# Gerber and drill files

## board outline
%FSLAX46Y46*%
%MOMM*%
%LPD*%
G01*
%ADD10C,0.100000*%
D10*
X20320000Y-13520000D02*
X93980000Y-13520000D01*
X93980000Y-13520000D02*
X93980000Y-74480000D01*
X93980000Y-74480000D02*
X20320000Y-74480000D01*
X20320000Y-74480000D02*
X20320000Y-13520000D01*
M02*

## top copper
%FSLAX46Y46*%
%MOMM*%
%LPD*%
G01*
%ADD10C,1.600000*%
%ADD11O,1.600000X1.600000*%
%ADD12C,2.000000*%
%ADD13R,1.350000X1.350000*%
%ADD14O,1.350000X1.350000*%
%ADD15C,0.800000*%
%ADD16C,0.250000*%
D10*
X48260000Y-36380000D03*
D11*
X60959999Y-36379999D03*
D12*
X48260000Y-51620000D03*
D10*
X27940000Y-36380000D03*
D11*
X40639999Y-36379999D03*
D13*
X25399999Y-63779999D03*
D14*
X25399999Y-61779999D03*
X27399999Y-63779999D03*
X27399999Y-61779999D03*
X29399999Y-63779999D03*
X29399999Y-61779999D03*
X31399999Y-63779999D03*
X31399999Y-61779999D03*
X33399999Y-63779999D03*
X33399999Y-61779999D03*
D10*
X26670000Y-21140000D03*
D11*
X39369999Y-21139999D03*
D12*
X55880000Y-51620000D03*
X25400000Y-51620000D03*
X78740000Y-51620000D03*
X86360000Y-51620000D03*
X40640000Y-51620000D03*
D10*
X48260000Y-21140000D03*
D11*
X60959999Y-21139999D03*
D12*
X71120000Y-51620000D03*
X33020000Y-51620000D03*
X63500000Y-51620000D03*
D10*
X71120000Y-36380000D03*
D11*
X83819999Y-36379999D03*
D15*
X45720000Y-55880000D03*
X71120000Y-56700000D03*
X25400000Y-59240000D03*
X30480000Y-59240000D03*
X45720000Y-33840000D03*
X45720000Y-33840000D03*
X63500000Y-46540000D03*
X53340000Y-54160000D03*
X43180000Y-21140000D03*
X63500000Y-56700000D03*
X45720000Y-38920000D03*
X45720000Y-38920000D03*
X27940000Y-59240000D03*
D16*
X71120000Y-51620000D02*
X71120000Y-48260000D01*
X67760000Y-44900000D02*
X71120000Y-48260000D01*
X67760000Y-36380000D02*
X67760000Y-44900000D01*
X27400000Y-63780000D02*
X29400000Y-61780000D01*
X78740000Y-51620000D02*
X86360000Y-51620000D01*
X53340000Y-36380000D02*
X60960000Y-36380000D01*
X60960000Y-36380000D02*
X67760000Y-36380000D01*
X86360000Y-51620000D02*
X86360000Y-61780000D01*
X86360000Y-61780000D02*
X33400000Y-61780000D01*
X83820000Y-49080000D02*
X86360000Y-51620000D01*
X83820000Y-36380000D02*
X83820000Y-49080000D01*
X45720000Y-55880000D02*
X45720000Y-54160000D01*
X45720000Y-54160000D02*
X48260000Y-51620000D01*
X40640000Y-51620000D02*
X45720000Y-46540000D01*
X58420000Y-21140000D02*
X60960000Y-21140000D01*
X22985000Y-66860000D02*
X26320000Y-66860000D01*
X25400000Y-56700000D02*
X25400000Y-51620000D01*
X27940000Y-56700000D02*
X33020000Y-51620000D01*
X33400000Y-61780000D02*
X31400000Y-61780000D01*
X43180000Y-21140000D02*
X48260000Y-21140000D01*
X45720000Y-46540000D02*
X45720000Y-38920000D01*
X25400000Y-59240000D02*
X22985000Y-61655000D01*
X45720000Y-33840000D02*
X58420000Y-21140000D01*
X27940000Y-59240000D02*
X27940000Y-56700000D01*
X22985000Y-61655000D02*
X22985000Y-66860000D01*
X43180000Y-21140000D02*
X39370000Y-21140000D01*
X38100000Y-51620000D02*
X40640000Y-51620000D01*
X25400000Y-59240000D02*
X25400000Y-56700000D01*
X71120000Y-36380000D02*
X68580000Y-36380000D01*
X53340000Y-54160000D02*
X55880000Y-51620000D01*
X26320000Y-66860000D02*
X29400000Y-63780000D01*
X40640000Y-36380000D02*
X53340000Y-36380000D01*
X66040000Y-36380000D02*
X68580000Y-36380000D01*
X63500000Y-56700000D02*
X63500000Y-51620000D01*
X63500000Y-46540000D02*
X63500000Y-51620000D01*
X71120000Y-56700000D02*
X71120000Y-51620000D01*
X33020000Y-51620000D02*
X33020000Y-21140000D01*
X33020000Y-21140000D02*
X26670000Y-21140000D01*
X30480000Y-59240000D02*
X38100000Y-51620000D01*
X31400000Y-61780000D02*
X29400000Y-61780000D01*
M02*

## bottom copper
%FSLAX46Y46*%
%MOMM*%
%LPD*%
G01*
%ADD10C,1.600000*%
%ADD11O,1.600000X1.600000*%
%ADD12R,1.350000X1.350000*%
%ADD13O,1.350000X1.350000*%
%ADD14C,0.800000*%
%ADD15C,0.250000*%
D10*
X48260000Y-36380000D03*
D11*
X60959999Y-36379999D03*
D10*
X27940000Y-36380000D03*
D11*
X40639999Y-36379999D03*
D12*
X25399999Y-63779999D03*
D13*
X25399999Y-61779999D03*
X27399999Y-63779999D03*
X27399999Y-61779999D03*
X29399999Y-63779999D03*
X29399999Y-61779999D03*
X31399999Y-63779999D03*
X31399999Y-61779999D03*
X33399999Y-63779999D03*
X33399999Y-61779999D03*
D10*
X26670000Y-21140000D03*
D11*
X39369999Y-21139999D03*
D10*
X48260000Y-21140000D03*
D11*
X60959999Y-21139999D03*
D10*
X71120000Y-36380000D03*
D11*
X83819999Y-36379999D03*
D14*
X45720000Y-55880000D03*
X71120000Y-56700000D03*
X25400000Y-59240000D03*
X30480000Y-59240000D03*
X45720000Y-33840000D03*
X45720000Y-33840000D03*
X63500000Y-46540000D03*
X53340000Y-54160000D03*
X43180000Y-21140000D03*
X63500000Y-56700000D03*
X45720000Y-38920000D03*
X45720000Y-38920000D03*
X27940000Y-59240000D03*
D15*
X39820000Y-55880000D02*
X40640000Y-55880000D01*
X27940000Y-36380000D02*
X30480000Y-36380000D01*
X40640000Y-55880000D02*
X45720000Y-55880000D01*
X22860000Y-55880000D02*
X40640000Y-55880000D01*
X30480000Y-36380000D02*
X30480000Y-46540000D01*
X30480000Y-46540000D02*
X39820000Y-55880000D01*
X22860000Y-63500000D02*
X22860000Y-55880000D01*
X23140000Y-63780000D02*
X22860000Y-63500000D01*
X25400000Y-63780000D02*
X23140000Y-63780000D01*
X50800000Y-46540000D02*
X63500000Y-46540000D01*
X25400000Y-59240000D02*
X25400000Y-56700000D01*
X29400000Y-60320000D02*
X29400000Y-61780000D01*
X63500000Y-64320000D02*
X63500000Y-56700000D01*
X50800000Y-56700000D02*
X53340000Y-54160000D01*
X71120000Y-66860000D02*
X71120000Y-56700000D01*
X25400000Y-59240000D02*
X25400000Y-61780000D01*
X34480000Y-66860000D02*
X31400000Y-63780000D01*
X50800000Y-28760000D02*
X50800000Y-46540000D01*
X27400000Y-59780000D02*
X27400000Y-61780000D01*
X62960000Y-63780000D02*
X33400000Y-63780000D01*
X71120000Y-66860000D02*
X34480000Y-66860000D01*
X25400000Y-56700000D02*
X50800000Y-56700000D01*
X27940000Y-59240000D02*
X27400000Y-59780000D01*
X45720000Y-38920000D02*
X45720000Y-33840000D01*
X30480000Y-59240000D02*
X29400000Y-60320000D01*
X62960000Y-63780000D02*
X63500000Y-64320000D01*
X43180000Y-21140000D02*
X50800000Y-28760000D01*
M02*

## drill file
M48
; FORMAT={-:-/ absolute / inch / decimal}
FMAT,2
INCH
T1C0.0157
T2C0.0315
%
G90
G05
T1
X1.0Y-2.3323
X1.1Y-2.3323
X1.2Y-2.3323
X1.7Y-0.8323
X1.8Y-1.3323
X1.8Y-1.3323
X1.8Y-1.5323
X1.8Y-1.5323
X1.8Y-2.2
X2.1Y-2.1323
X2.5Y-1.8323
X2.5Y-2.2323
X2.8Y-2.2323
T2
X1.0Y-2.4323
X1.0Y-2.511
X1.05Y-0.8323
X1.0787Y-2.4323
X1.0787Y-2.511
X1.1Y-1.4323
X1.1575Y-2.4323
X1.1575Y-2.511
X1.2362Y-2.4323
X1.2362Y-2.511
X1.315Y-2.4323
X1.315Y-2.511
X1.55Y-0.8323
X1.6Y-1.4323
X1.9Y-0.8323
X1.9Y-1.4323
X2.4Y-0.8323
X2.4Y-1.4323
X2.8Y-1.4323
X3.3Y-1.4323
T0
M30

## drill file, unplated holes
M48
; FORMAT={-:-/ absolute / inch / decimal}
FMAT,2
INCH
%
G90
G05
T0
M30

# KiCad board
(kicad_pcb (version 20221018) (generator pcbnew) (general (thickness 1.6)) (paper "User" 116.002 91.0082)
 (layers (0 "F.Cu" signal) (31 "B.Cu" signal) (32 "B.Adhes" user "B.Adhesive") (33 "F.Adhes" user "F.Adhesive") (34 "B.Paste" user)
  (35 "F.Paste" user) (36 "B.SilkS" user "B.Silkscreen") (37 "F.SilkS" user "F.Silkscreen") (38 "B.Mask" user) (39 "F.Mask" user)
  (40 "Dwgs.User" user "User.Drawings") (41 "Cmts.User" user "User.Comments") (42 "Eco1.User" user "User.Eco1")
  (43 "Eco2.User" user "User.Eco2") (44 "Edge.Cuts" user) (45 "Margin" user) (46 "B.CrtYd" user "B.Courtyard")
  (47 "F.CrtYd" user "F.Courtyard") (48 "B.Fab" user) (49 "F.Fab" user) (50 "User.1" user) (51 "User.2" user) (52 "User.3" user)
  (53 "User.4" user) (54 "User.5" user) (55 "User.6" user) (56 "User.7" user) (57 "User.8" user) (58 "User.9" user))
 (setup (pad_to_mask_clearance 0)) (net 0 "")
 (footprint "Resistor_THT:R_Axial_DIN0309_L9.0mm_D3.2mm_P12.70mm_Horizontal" (layer "F.Cu") (at 27.94 36.38)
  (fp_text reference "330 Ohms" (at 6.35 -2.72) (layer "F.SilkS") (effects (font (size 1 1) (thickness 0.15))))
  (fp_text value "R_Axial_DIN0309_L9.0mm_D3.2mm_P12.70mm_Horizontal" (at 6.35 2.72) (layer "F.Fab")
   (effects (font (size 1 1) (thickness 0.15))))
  (pad "1" thru_hole circle (at 0 0) (size 1.6 1.6) (drill 0.8) (layers "*.Cu" "*.Mask"))
  (pad "2" thru_hole oval (at 12.7 0) (size 1.6 1.6) (drill 0.8) (layers "*.Cu" "*.Mask")))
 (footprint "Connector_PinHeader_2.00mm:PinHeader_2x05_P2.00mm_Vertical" (layer "F.Cu") (at 25.4 63.78 90)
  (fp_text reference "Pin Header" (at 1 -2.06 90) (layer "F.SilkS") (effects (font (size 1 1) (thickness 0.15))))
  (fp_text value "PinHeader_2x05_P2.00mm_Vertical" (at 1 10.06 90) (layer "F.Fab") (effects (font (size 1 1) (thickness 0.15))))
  (pad "1" thru_hole rect (at 0 0 90) (size 1.35 1.35) (drill 0.8) (layers "*.Cu" "*.Mask"))
  (pad "2" thru_hole oval (at 2 0 90) (size 1.35 1.35) (drill 0.8) (layers "*.Cu" "*.Mask"))
  (pad "3" thru_hole oval (at 0 2 90) (size 1.35 1.35) (drill 0.8) (layers "*.Cu" "*.Mask"))
  (pad "4" thru_hole oval (at 2 2 90) (size 1.35 1.35) (drill 0.8) (layers "*.Cu" "*.Mask"))
  (pad "5" thru_hole oval (at 0 4 90) (size 1.35 1.35) (drill 0.8) (layers "*.Cu" "*.Mask"))
  (pad "6" thru_hole oval (at 2 4 90) (size 1.35 1.35) (drill 0.8) (layers "*.Cu" "*.Mask"))
  (pad "7" thru_hole oval (at 0 6 90) (size 1.35 1.35) (drill 0.8) (layers "*.Cu" "*.Mask"))
  (pad "8" thru_hole oval (at 2 6 90) (size 1.35 1.35) (drill 0.8) (layers "*.Cu" "*.Mask"))
  (pad "9" thru_hole oval (at 0 8 90) (size 1.35 1.35) (drill 0.8) (layers "*.Cu" "*.Mask"))
  (pad "10" thru_hole oval (at 2 8 90) (size 1.35 1.35) (drill 0.8) (layers "*.Cu" "*.Mask")))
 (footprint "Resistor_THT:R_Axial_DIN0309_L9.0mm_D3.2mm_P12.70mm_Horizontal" (layer "F.Cu") (at 26.67 21.14)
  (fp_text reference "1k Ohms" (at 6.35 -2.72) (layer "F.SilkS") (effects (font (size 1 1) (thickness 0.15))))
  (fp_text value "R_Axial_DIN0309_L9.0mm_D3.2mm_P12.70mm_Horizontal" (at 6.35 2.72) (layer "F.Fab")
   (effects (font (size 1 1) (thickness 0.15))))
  (pad "1" thru_hole circle (at 0 0) (size 1.6 1.6) (drill 0.8) (layers "*.Cu" "*.Mask"))
  (pad "2" thru_hole oval (at 12.7 0) (size 1.6 1.6) (drill 0.8) (layers "*.Cu" "*.Mask")))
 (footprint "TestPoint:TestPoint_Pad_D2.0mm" (layer "F.Cu") (at 55.88 51.62)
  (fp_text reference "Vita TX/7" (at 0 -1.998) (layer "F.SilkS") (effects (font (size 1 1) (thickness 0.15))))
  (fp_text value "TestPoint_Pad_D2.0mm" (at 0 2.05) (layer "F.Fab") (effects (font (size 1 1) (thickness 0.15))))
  (pad "1" smd circle (at 0 0) (size 2 2) (layers "F.Cu" "F.Mask")))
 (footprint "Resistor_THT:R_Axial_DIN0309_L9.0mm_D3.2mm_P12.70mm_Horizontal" (layer "F.Cu") (at 48.26 36.38)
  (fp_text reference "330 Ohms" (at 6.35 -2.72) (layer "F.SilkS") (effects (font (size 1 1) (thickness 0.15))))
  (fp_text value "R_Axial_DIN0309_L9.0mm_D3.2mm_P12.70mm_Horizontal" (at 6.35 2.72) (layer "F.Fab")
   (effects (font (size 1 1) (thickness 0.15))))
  (pad "1" thru_hole circle (at 0 0) (size 1.6 1.6) (drill 0.8) (layers "*.Cu" "*.Mask"))
  (pad "2" thru_hole oval (at 12.7 0) (size 1.6 1.6) (drill 0.8) (layers "*.Cu" "*.Mask")))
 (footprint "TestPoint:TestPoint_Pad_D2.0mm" (layer "F.Cu") (at 48.26 51.62)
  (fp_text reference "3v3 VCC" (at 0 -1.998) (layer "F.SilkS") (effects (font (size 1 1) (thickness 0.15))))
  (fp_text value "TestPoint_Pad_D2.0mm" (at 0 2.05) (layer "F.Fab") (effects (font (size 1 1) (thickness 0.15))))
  (pad "1" smd circle (at 0 0) (size 2 2) (layers "F.Cu" "F.Mask")))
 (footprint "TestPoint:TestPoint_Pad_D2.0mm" (layer "F.Cu") (at 25.4 51.62)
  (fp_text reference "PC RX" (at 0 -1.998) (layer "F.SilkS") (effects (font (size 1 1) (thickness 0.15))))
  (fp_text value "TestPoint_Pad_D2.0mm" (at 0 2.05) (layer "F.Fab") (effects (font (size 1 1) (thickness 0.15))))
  (pad "1" smd circle (at 0 0) (size 2 2) (layers "F.Cu" "F.Mask")))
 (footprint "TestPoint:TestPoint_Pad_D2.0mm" (layer "F.Cu") (at 78.74 51.62)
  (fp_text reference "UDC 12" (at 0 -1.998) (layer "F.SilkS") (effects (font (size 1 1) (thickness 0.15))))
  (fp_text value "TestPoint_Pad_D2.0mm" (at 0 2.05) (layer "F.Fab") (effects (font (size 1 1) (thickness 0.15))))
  (pad "1" smd circle (at 0 0) (size 2 2) (layers "F.Cu" "F.Mask")))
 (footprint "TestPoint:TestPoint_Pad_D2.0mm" (layer "F.Cu") (at 86.36 51.62)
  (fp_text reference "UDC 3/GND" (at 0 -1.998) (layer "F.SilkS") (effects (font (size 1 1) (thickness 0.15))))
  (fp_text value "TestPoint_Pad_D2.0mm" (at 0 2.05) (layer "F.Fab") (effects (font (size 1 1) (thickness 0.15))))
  (pad "1" smd circle (at 0 0) (size 2 2) (layers "F.Cu" "F.Mask")))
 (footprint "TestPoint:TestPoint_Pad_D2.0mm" (layer "F.Cu") (at 40.64 51.62)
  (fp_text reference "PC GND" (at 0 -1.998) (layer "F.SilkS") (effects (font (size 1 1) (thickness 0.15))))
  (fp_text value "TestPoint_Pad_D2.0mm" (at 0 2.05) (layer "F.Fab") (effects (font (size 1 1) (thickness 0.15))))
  (pad "1" smd circle (at 0 0) (size 2 2) (layers "F.Cu" "F.Mask")))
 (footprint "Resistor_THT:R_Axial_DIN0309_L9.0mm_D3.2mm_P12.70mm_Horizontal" (layer "F.Cu") (at 48.26 21.14)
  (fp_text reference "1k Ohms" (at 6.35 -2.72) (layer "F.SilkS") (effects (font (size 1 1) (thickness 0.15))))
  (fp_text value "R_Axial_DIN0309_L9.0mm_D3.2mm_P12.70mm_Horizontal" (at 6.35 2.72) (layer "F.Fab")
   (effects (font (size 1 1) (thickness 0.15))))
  (pad "1" thru_hole circle (at 0 0) (size 1.6 1.6) (drill 0.8) (layers "*.Cu" "*.Mask"))
  (pad "2" thru_hole oval (at 12.7 0) (size 1.6 1.6) (drill 0.8) (layers "*.Cu" "*.Mask")))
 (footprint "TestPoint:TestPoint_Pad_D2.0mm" (layer "F.Cu") (at 71.12 51.62)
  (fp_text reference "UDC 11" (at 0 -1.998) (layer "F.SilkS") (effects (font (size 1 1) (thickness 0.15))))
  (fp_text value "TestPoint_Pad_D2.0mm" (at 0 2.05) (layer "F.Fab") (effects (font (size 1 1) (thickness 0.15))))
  (pad "1" smd circle (at 0 0) (size 2 2) (layers "F.Cu" "F.Mask")))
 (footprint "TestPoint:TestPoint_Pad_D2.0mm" (layer "F.Cu") (at 33.02 51.62)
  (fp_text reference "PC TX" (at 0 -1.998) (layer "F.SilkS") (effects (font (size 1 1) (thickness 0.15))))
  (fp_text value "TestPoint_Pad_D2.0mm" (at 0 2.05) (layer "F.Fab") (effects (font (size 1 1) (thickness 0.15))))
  (pad "1" smd circle (at 0 0) (size 2 2) (layers "F.Cu" "F.Mask")))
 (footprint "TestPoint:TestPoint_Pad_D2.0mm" (layer "F.Cu") (at 63.5 51.62)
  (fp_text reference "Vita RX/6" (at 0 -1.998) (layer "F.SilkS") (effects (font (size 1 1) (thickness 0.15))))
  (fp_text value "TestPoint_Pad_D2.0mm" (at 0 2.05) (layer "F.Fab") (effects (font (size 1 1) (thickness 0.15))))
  (pad "1" smd circle (at 0 0) (size 2 2) (layers "F.Cu" "F.Mask")))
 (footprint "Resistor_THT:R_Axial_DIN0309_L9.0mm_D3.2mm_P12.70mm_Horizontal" (layer "F.Cu") (at 71.12 36.38)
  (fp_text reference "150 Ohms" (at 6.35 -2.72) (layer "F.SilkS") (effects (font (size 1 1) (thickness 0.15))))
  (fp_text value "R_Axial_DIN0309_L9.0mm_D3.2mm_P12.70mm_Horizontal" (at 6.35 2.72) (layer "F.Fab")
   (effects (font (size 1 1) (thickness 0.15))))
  (pad "1" thru_hole circle (at 0 0) (size 1.6 1.6) (drill 0.8) (layers "*.Cu" "*.Mask"))
  (pad "2" thru_hole oval (at 12.7 0) (size 1.6 1.6) (drill 0.8) (layers "*.Cu" "*.Mask")))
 (gr_rect (start 20.32 13.52) (end 93.98 74.48) (stroke (width 0.1) (type default)) (fill none) (layer "Edge.Cuts"))
 (segment (start 67.76 36.38) (end 67.76 44.9) (width 0.25) (layer "F.Cu") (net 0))
 (segment (start 40.64 51.62) (end 45.72 46.54) (width 0.25) (layer "F.Cu") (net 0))
 (segment (start 58.42 21.14) (end 60.96 21.14) (width 0.25) (layer "F.Cu") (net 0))
 (segment (start 22.985 66.86) (end 26.32 66.86) (width 0.25) (layer "F.Cu") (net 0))
 (segment (start 25.4 56.7) (end 25.4 51.62) (width 0.25) (layer "F.Cu") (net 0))
 (segment (start 83.82 49.08) (end 86.36 51.62) (width 0.25) (layer "F.Cu") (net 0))
 (segment (start 27.94 56.7) (end 33.02 51.62) (width 0.25) (layer "F.Cu") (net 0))
 (segment (start 33.4 61.78) (end 31.4 61.78) (width 0.25) (layer "F.Cu") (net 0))
 (segment (start 43.18 21.14) (end 48.26 21.14) (width 0.25) (layer "F.Cu") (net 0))
 (segment (start 45.72 46.54) (end 45.72 38.92) (width 0.25) (layer "F.Cu") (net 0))
 (segment (start 45.72 55.88) (end 45.72 54.16) (width 0.25) (layer "F.Cu") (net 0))
 (segment (start 60.96 36.38) (end 67.76 36.38) (width 0.25) (layer "F.Cu") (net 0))
 (segment (start 25.4 59.24) (end 22.985 61.655) (width 0.25) (layer "F.Cu") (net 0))
 (segment (start 67.76 44.9) (end 71.12 48.26) (width 0.25) (layer "F.Cu") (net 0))
 (segment (start 45.72 54.16) (end 48.26 51.62) (width 0.25) (layer "F.Cu") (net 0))
 (segment (start 45.72 33.84) (end 58.42 21.14) (width 0.25) (layer "F.Cu") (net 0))
 (segment (start 27.94 59.24) (end 27.94 56.7) (width 0.25) (layer "F.Cu") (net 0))
 (segment (start 22.985 61.655) (end 22.985 66.86) (width 0.25) (layer "F.Cu") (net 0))
 (segment (start 43.18 21.14) (end 39.37 21.14) (width 0.25) (layer "F.Cu") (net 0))
 (segment (start 38.1 51.62) (end 40.64 51.62) (width 0.25) (layer "F.Cu") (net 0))
 (segment (start 25.4 59.24) (end 25.4 56.7) (width 0.25) (layer "F.Cu") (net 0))
 (segment (start 78.74 51.62) (end 86.36 51.62) (width 0.25) (layer "F.Cu") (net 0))
 (segment (start 71.12 36.38) (end 68.58 36.38) (width 0.25) (layer "F.Cu") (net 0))
 (segment (start 53.34 54.16) (end 55.88 51.62) (width 0.25) (layer "F.Cu") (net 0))
 (segment (start 26.32 66.86) (end 29.4 63.78) (width 0.25) (layer "F.Cu") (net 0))
 (segment (start 40.64 36.38) (end 53.34 36.38) (width 0.25) (layer "F.Cu") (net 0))
 (segment (start 86.36 61.78) (end 33.4 61.78) (width 0.25) (layer "F.Cu") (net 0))
 (segment (start 27.4 63.78) (end 29.4 61.78) (width 0.25) (layer "F.Cu") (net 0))
 (segment (start 53.34 36.38) (end 60.96 36.38) (width 0.25) (layer "F.Cu") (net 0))
 (segment (start 66.04 36.38) (end 68.58 36.38) (width 0.25) (layer "F.Cu") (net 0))
 (segment (start 83.82 36.38) (end 83.82 49.08) (width 0.25) (layer "F.Cu") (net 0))
 (segment (start 63.5 56.7) (end 63.5 51.62) (width 0.25) (layer "F.Cu") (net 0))
 (segment (start 63.5 46.54) (end 63.5 51.62) (width 0.25) (layer "F.Cu") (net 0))
 (segment (start 71.12 56.7) (end 71.12 51.62) (width 0.25) (layer "F.Cu") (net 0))
 (segment (start 33.02 51.62) (end 33.02 21.14) (width 0.25) (layer "F.Cu") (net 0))
 (segment (start 33.02 21.14) (end 26.67 21.14) (width 0.25) (layer "F.Cu") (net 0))
 (segment (start 86.36 51.62) (end 86.36 61.78) (width 0.25) (layer "F.Cu") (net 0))
 (segment (start 71.12 51.62) (end 71.12 48.26) (width 0.25) (layer "F.Cu") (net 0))
 (segment (start 30.48 59.24) (end 38.1 51.62) (width 0.25) (layer "F.Cu") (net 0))
 (segment (start 31.4 61.78) (end 29.4 61.78) (width 0.25) (layer "F.Cu") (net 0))
 (via (at 71.12 56.7) (size 0.8) (drill 0.4) (layers "F.Cu" "B.Cu") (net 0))
 (via (at 25.4 59.24) (size 0.8) (drill 0.4) (layers "F.Cu" "B.Cu") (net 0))
 (via (at 30.48 59.24) (size 0.8) (drill 0.4) (layers "F.Cu" "B.Cu") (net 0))
 (via (at 45.72 33.84) (size 0.8) (drill 0.4) (layers "F.Cu" "B.Cu") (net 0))
 (via (at 45.72 33.84) (size 0.8) (drill 0.4) (layers "F.Cu" "B.Cu") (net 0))
 (via (at 63.5 46.54) (size 0.8) (drill 0.4) (layers "F.Cu" "B.Cu") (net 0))
 (via (at 53.34 54.16) (size 0.8) (drill 0.4) (layers "F.Cu" "B.Cu") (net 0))
 (via (at 43.18 21.14) (size 0.8) (drill 0.4) (layers "F.Cu" "B.Cu") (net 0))
 (via (at 63.5 56.7) (size 0.8) (drill 0.4) (layers "F.Cu" "B.Cu") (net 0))
 (via (at 45.72 38.92) (size 0.8) (drill 0.4) (layers "F.Cu" "B.Cu") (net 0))
 (via (at 45.72 38.92) (size 0.8) (drill 0.4) (layers "F.Cu" "B.Cu") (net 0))
 (via (at 27.94 59.24) (size 0.8) (drill 0.4) (layers "F.Cu" "B.Cu") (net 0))
 (via (at 45.72 55.88) (size 0.8) (drill 0.4) (layers "F.Cu" "B.Cu") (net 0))
 (segment (start 27.94 36.38) (end 30.48 36.38) (width 0.25) (layer "B.Cu") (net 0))
 (segment (start 50.8 46.54) (end 63.5 46.54) (width 0.25) (layer "B.Cu") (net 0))
 (segment (start 40.64 55.88) (end 45.72 55.88) (width 0.25) (layer "B.Cu") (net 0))
 (segment (start 25.4 59.24) (end 25.4 56.7) (width 0.25) (layer "B.Cu") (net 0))
 (segment (start 30.48 46.54) (end 39.82 55.88) (width 0.25) (layer "B.Cu") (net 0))
 (segment (start 29.4 60.32) (end 29.4 61.78) (width 0.25) (layer "B.Cu") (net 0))
 (segment (start 63.5 64.32) (end 63.5 56.7) (width 0.25) (layer "B.Cu") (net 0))
 (segment (start 22.86 55.88) (end 40.64 55.88) (width 0.25) (layer "B.Cu") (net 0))
 (segment (start 25.4 63.78) (end 23.14 63.78) (width 0.25) (layer "B.Cu") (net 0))
 (segment (start 50.8 56.7) (end 53.34 54.16) (width 0.25) (layer "B.Cu") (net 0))
 (segment (start 71.12 66.86) (end 71.12 56.7) (width 0.25) (layer "B.Cu") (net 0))
 (segment (start 25.4 59.24) (end 25.4 61.78) (width 0.25) (layer "B.Cu") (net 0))
 (segment (start 23.14 63.78) (end 22.86 63.5) (width 0.25) (layer "B.Cu") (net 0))
 (segment (start 34.48 66.86) (end 31.4 63.78) (width 0.25) (layer "B.Cu") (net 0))
 (segment (start 50.8 28.76) (end 50.8 46.54) (width 0.25) (layer "B.Cu") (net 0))
 (segment (start 27.4 59.78) (end 27.4 61.78) (width 0.25) (layer "B.Cu") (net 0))
 (segment (start 22.86 63.5) (end 22.86 55.88) (width 0.25) (layer "B.Cu") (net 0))
 (segment (start 62.96 63.78) (end 33.4 63.78) (width 0.25) (layer "B.Cu") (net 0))
 (segment (start 71.12 66.86) (end 34.48 66.86) (width 0.25) (layer "B.Cu") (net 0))
 (segment (start 25.4 56.7) (end 50.8 56.7) (width 0.25) (layer "B.Cu") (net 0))
 (segment (start 30.48 36.38) (end 30.48 46.54) (width 0.25) (layer "B.Cu") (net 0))
 (segment (start 39.82 55.88) (end 40.64 55.88) (width 0.25) (layer "B.Cu") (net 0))
 (segment (start 27.94 59.24) (end 27.4 59.78) (width 0.25) (layer "B.Cu") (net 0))
 (segment (start 45.72 38.92) (end 45.72 33.84) (width 0.25) (layer "B.Cu") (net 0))
 (segment (start 30.48 59.24) (end 29.4 60.32) (width 0.25) (layer "B.Cu") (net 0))
 (segment (start 62.96 63.78) (end 63.5 64.32) (width 0.25) (layer "B.Cu") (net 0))
 (segment (start 43.18 21.14) (end 50.8 28.76) (width 0.25) (layer "B.Cu") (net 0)))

